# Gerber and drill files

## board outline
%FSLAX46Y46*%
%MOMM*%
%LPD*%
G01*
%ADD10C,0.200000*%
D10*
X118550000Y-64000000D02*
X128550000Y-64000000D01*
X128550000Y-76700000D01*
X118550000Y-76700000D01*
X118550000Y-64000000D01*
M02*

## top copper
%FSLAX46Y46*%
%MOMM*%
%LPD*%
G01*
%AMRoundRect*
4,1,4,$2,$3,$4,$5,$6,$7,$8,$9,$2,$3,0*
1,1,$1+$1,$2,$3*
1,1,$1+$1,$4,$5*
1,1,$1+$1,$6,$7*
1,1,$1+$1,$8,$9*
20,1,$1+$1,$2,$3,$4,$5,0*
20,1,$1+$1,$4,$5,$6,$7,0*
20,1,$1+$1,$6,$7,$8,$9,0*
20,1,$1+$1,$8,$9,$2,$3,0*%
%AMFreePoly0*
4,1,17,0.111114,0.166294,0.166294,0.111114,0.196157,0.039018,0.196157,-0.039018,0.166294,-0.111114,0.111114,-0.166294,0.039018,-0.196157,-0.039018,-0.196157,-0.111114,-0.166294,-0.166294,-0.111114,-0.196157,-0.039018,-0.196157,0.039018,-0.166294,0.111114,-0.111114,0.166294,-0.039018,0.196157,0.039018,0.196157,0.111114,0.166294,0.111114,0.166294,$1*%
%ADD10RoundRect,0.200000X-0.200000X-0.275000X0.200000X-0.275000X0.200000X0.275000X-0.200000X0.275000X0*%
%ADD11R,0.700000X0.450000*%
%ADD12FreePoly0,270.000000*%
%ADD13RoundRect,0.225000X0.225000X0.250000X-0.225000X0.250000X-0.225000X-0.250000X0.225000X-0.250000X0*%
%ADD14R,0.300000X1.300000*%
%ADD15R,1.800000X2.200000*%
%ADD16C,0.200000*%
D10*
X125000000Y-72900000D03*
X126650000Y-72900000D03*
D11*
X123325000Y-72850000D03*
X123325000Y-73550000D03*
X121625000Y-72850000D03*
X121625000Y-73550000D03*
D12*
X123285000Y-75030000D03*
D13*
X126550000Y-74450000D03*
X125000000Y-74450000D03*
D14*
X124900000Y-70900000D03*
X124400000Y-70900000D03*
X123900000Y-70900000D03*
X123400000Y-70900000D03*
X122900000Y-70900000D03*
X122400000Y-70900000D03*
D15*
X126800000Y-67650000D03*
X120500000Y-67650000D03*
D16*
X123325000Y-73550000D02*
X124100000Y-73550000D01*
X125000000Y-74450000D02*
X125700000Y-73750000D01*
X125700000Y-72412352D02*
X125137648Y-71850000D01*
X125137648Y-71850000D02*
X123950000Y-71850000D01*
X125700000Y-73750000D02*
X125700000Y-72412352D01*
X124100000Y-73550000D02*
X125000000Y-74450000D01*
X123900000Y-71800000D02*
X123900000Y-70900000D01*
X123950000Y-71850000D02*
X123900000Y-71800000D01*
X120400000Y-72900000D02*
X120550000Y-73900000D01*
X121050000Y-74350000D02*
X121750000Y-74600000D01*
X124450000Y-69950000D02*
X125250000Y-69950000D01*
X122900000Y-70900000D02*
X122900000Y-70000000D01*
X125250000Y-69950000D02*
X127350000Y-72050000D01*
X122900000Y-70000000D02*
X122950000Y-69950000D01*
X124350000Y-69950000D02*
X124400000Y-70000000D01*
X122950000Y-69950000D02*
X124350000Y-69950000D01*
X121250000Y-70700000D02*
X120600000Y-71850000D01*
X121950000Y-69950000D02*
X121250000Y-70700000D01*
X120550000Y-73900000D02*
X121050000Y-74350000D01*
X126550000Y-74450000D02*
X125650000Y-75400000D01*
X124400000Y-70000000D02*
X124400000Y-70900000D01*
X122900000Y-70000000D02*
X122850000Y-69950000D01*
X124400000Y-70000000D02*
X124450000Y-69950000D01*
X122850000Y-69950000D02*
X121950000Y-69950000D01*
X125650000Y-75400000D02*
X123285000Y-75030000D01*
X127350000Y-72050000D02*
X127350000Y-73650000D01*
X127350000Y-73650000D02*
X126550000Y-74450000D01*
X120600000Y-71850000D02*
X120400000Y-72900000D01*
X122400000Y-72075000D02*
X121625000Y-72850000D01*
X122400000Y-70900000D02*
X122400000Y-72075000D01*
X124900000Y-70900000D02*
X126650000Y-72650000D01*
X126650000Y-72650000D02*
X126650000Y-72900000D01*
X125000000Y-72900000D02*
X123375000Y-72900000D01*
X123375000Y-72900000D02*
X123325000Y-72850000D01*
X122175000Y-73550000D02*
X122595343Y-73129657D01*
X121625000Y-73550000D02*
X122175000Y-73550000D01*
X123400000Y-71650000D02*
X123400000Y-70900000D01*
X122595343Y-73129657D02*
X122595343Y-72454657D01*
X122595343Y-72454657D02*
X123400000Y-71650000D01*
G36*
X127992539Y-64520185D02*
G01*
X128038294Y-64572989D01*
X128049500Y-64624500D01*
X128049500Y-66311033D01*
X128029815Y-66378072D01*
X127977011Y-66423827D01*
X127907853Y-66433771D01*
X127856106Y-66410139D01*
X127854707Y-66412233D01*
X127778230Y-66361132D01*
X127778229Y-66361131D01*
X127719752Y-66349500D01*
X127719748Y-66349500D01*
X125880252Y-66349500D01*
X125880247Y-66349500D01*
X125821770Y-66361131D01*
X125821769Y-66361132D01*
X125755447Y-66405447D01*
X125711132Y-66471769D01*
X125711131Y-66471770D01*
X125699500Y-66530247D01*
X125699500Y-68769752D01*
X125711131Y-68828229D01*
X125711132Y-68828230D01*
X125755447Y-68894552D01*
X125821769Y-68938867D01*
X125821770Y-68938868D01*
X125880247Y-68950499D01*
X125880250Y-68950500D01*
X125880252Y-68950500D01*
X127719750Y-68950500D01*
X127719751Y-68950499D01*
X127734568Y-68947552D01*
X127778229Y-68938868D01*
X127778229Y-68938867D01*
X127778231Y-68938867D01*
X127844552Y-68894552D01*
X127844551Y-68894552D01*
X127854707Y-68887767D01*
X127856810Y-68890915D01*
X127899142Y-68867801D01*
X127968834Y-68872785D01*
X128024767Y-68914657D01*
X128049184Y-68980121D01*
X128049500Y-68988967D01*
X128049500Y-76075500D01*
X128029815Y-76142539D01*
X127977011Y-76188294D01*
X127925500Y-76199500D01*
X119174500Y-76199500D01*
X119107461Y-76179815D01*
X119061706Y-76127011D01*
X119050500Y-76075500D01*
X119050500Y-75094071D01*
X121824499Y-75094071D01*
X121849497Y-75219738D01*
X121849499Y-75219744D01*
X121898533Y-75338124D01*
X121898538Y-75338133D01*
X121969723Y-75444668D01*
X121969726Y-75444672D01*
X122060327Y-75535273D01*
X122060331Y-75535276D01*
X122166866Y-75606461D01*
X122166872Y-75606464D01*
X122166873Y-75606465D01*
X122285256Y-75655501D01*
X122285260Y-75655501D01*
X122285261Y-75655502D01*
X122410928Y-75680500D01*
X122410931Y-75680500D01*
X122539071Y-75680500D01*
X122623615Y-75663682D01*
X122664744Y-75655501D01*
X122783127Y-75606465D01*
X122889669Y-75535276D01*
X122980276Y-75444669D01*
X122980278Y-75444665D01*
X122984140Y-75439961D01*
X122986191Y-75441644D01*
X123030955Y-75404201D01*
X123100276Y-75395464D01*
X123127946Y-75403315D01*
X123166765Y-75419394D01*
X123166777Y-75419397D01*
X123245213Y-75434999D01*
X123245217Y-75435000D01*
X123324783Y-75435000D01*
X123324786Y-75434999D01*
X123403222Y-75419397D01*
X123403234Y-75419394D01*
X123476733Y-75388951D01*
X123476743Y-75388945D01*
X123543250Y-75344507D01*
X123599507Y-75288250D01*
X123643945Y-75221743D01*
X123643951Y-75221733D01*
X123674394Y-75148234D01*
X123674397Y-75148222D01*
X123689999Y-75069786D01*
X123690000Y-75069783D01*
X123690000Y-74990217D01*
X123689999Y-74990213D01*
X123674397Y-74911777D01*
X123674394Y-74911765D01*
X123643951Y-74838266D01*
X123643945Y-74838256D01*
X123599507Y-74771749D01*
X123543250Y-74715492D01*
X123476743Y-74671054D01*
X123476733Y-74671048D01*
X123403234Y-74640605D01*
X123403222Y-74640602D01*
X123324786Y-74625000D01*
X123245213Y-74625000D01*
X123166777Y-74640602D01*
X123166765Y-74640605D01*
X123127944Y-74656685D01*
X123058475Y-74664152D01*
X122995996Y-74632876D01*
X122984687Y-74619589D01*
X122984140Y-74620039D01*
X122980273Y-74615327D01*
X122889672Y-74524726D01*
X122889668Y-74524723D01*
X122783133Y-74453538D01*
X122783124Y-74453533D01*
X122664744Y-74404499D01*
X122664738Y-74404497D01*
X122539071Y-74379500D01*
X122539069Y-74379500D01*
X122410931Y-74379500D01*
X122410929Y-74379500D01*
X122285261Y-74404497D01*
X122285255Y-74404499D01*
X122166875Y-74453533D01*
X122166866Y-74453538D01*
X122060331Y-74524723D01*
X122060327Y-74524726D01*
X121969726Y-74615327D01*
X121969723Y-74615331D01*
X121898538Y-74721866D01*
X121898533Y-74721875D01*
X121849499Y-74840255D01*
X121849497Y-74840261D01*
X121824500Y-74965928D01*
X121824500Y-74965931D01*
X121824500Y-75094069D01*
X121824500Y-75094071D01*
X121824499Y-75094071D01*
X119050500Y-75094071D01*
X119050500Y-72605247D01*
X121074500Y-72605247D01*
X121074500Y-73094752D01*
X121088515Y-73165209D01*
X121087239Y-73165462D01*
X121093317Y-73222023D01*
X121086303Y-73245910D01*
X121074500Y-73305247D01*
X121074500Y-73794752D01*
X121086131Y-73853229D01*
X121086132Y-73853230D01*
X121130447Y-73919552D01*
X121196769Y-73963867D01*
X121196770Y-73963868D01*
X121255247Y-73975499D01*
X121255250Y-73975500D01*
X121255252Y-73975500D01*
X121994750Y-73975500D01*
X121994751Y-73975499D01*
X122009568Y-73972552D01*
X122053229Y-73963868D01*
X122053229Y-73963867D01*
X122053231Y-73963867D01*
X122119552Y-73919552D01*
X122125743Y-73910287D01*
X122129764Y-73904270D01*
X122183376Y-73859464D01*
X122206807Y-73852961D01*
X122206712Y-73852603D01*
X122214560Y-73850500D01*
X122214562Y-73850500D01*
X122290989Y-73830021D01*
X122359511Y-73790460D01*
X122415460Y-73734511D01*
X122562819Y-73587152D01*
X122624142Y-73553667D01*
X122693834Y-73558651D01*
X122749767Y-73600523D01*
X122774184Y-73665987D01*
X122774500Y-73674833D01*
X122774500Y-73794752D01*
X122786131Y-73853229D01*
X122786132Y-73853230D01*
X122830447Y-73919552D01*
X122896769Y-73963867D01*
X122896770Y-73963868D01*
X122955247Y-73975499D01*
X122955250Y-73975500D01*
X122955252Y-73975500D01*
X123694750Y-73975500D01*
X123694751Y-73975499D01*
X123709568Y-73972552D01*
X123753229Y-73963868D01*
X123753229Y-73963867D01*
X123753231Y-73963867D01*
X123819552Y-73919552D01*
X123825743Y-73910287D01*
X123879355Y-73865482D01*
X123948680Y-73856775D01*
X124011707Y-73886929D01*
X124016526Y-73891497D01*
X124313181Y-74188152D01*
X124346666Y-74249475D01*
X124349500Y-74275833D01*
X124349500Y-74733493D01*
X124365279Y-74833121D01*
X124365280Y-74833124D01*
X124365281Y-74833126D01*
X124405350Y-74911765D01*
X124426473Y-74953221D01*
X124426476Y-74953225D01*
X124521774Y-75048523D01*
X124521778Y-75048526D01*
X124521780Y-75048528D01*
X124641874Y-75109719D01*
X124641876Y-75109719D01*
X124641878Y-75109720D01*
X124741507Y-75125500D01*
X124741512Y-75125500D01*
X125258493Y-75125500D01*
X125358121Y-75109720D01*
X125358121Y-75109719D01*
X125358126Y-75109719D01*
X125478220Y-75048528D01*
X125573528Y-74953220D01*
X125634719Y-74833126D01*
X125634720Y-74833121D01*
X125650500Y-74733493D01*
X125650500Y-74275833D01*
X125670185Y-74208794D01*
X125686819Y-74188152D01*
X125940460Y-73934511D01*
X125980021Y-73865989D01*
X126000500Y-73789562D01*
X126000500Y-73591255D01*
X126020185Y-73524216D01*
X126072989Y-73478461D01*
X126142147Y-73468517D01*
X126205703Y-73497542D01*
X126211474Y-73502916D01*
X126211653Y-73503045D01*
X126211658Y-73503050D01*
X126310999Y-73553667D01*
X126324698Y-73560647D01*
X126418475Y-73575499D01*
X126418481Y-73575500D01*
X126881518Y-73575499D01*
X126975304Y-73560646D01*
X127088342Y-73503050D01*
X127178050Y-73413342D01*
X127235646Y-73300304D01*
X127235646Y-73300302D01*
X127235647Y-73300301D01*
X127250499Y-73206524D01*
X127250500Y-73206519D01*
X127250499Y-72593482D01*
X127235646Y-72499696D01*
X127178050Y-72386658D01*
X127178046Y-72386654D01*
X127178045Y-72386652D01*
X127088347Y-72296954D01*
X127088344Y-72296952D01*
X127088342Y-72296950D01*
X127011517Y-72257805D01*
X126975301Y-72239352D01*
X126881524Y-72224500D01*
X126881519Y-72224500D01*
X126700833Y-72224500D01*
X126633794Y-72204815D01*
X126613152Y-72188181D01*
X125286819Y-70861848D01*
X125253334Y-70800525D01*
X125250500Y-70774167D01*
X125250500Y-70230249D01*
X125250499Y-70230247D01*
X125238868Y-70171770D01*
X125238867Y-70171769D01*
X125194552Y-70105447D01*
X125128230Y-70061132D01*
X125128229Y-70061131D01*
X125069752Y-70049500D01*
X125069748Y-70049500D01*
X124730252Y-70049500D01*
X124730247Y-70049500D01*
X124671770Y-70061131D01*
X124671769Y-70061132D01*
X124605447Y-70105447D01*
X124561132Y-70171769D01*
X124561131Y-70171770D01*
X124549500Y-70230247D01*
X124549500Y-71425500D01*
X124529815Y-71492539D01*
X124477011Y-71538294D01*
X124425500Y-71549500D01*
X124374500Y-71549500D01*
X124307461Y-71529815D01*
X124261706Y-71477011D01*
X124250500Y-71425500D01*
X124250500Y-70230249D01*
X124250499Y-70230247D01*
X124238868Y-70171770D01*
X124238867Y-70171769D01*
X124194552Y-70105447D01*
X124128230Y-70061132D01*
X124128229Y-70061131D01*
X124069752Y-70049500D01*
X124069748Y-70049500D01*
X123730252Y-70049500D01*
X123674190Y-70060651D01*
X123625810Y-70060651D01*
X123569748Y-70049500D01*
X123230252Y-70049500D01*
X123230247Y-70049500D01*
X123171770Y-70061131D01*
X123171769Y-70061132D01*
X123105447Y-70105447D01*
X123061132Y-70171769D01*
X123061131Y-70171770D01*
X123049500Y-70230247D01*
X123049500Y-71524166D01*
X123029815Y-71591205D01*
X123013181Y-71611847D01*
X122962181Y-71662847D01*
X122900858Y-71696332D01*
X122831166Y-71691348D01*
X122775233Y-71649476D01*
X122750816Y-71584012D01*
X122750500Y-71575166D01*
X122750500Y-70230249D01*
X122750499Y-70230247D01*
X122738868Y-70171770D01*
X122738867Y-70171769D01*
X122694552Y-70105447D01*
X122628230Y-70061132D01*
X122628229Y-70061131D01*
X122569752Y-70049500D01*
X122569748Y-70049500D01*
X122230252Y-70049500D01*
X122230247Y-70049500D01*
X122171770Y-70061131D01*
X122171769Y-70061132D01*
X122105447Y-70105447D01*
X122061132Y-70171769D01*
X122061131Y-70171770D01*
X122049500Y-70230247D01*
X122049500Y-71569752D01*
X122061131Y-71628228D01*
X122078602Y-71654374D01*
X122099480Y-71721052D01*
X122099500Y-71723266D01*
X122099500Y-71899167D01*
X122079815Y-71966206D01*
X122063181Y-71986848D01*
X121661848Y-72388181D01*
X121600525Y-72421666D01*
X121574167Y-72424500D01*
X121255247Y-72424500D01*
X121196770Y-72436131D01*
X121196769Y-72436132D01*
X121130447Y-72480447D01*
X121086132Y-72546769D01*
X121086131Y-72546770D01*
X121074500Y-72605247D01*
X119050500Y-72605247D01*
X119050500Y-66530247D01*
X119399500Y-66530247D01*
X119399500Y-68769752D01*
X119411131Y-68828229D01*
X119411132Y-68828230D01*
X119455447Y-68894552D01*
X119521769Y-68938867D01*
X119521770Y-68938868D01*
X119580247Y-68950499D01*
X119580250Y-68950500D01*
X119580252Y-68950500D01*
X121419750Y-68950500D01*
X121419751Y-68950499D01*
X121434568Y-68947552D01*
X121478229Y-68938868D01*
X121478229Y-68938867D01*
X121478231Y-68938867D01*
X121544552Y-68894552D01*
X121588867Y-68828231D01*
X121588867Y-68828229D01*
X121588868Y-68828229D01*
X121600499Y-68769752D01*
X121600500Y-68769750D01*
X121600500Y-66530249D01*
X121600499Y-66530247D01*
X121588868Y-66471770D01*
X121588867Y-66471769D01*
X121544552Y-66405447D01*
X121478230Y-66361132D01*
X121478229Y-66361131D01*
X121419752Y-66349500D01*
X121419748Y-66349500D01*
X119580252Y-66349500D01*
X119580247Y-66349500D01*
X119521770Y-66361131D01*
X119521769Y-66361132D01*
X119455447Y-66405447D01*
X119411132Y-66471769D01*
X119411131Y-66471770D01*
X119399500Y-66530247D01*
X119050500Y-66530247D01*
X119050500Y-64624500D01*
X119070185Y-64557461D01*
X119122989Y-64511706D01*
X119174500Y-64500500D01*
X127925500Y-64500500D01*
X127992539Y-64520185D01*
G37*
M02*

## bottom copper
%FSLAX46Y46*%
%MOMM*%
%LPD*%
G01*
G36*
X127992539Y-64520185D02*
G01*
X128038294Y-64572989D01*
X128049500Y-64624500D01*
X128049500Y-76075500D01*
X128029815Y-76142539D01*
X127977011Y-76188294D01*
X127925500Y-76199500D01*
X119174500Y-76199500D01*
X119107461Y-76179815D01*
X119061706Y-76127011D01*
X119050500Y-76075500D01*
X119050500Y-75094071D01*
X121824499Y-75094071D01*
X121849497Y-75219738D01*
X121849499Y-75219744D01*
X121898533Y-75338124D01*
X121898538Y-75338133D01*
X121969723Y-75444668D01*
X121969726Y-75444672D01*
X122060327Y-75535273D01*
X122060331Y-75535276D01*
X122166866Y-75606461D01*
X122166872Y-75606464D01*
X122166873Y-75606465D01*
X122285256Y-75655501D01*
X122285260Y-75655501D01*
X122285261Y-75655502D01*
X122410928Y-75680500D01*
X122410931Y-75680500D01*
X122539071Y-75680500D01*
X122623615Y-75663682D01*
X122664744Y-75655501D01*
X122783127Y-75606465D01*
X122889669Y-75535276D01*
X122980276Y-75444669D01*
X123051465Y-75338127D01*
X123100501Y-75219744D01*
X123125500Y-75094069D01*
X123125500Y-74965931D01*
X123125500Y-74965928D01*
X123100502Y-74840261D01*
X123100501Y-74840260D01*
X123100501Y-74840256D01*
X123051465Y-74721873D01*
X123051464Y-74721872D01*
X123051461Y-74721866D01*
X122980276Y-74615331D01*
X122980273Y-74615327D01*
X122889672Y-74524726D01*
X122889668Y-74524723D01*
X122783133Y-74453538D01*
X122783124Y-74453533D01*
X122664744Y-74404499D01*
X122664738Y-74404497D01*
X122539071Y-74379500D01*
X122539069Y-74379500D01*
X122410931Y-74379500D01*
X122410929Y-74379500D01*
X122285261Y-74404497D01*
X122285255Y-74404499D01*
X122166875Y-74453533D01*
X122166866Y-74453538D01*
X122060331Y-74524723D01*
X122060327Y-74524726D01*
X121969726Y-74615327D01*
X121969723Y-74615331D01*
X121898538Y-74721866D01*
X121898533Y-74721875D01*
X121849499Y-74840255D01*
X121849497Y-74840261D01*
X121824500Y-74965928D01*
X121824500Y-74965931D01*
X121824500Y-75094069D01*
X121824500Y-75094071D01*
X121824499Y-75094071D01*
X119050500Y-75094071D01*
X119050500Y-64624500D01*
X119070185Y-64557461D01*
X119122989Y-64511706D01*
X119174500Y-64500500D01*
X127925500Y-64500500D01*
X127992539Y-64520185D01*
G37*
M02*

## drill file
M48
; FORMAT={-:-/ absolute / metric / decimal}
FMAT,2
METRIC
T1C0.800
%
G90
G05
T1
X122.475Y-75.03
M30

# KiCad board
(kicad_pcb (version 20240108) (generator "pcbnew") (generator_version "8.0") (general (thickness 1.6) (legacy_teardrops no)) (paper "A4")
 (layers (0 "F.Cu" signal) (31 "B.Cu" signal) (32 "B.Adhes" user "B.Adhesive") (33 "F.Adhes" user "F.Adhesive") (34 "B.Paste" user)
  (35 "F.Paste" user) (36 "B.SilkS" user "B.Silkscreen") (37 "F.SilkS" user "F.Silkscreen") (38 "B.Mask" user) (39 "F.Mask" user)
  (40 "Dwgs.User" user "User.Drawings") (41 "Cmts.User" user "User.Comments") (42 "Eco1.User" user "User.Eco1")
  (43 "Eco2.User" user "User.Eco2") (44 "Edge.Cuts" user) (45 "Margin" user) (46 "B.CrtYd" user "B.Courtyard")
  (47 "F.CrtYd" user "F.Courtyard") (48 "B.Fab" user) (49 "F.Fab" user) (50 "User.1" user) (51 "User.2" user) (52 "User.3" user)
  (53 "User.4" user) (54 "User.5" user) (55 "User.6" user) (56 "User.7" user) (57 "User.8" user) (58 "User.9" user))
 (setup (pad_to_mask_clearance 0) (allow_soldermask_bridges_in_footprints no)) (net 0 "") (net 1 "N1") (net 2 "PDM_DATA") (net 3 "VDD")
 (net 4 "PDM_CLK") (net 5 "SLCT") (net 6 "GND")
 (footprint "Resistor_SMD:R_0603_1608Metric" (layer "F.Cu") (at 125.825 72.9)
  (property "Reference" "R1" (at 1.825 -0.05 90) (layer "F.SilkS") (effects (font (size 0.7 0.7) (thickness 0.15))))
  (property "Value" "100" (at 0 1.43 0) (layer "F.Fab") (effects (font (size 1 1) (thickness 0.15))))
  (pad "1" smd roundrect (at -0.825 0) (size 0.8 0.95) (layers "F.Cu" "F.Paste" "F.Mask") (roundrect_rratio 0.25) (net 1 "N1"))
  (pad "2" smd roundrect (at 0.825 0) (size 0.8 0.95) (layers "F.Cu" "F.Paste" "F.Mask") (roundrect_rratio 0.25) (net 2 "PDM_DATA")))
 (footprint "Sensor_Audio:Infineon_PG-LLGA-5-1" (layer "F.Cu") (at 122.475 74.35 -90)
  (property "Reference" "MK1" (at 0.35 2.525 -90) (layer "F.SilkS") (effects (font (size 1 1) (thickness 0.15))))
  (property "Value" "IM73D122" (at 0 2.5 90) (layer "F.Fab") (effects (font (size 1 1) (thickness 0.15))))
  (pad "" smd custom (at -1.5 -0.725 270) (size 0.3 0.3) (layers "F.Paste") (zone_connect 0) (options (clearance outline) (anchor circle))
   (primitives))
  (pad "" smd custom (at -1.5 0.725 270) (size 0.3 0.3) (layers "F.Paste") (zone_connect 0) (options (clearance outline) (anchor circle))
   (primitives))
  (pad "" smd custom (at -0.8 -0.725 270) (size 0.3 0.3) (layers "F.Paste") (zone_connect 0) (options (clearance outline) (anchor circle))
   (primitives))
  (pad "" smd custom (at -0.8 0.725 270) (size 0.3 0.3) (layers "F.Paste") (zone_connect 0) (options (clearance outline) (anchor circle))
   (primitives))
  (pad "" smd custom (at -0.12 0 270) (size 0.3 0.3) (layers "F.Paste") (zone_connect 0) (options (clearance outline) (anchor circle))
   (primitives))
  (pad "" smd custom (at 0.28 -0.693 270) (size 0.3 0.3) (layers "F.Paste") (zone_connect 0) (options (clearance outline) (anchor circle))
   (primitives))
  (pad "" smd custom (at 0.28 0.693 270) (size 0.3 0.3) (layers "F.Paste") (zone_connect 0) (options (clearance outline) (anchor circle))
   (primitives))
  (pad "" np_thru_hole circle (at 0.68 0 270) (size 0.8 0.8) (drill 0.8) (layers "*.Cu" "*.Mask"))
  (pad "" smd custom (at 1.08 -0.693 270) (size 0.3 0.3) (layers "F.Paste") (zone_connect 0) (options (clearance outline) (anchor circle))
   (primitives))
  (pad "" smd custom (at 1.08 0.693 270) (size 0.3 0.3) (layers "F.Paste") (zone_connect 0) (options (clearance outline) (anchor circle))
   (primitives))
  (pad "" smd custom (at 1.48 0 270) (size 0.3 0.3) (layers "F.Paste") (zone_connect 0) (options (clearance outline) (anchor circle))
   (primitives))
  (pad "1" smd rect (at -1.5 -0.85 270) (size 0.45 0.7) (layers "F.Cu" "F.Mask") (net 1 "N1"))
  (pad "2" smd rect (at -0.8 -0.85 270) (size 0.45 0.7) (layers "F.Cu" "F.Mask") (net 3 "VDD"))
  (pad "3" smd rect (at -1.5 0.85 270) (size 0.45 0.7) (layers "F.Cu" "F.Mask") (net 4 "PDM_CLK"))
  (pad "4" smd rect (at -0.8 0.85 270) (size 0.45 0.7) (layers "F.Cu" "F.Mask") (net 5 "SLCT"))
  (pad "5" smd custom (at 0.68 -0.81 270) (size 0.4 0.4) (layers "F.Cu" "F.Mask") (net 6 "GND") (zone_connect 0)
   (options (clearance outline) (anchor circle)) (primitives)))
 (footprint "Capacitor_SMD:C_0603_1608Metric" (layer "F.Cu") (at 125.775 74.45 180)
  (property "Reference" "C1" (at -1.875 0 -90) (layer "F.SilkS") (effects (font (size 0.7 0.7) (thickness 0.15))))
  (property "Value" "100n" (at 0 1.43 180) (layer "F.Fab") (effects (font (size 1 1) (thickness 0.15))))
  (pad "1" smd roundrect (at -0.775 0 180) (size 0.9 0.95) (layers "F.Cu" "F.Paste" "F.Mask") (roundrect_rratio 0.25) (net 6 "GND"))
  (pad "2" smd roundrect (at 0.775 0 180) (size 0.9 0.95) (layers "F.Cu" "F.Paste" "F.Mask") (roundrect_rratio 0.25) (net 3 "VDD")))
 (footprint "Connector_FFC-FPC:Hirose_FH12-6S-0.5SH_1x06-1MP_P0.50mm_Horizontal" (layer "F.Cu") (at 123.65 69.05 180)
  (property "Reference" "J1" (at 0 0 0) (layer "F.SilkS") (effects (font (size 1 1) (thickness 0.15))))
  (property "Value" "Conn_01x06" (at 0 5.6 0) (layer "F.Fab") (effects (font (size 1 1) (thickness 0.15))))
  (pad "1" smd rect (at -1.25 -1.85 180) (size 0.3 1.3) (layers "F.Cu" "F.Paste" "F.Mask") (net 2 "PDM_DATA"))
  (pad "2" smd rect (at -0.75 -1.85 180) (size 0.3 1.3) (layers "F.Cu" "F.Paste" "F.Mask") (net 6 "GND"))
  (pad "3" smd rect (at -0.25 -1.85 180) (size 0.3 1.3) (layers "F.Cu" "F.Paste" "F.Mask") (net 3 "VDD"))
  (pad "4" smd rect (at 0.25 -1.85 180) (size 0.3 1.3) (layers "F.Cu" "F.Paste" "F.Mask") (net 5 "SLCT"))
  (pad "5" smd rect (at 0.75 -1.85 180) (size 0.3 1.3) (layers "F.Cu" "F.Paste" "F.Mask") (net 6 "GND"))
  (pad "6" smd rect (at 1.25 -1.85 180) (size 0.3 1.3) (layers "F.Cu" "F.Paste" "F.Mask") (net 4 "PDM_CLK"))
  (pad "MP" smd rect (at -3.15 1.4 180) (size 1.8 2.2) (layers "F.Cu" "F.Paste" "F.Mask"))
  (pad "MP" smd rect (at 3.15 1.4 180) (size 1.8 2.2) (layers "F.Cu" "F.Paste" "F.Mask")))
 (gr_rect (start 118.55 64) (end 128.55 76.7) (stroke (width 0.2) (type default)) (fill none) (layer "Edge.Cuts"))
 (segment (start 123.325 73.55) (end 124.1 73.55) (width 0.2) (layer "F.Cu") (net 3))
 (segment (start 125 74.45) (end 125.7 73.75) (width 0.2) (layer "F.Cu") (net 3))
 (segment (start 125.7 72.412352) (end 125.137648 71.85) (width 0.2) (layer "F.Cu") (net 3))
 (segment (start 125.137648 71.85) (end 123.95 71.85) (width 0.2) (layer "F.Cu") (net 3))
 (segment (start 125.7 73.75) (end 125.7 72.412352) (width 0.2) (layer "F.Cu") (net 3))
 (segment (start 124.1 73.55) (end 125 74.45) (width 0.2) (layer "F.Cu") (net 3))
 (segment (start 123.9 71.8) (end 123.9 70.9) (width 0.2) (layer "F.Cu") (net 3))
 (segment (start 123.95 71.85) (end 123.9 71.8) (width 0.2) (layer "F.Cu") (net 3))
 (segment (start 120.4 72.9) (end 120.55 73.9) (width 0.2) (layer "F.Cu") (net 6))
 (segment (start 121.05 74.35) (end 121.75 74.6) (width 0.2) (layer "F.Cu") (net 6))
 (segment (start 124.45 69.95) (end 125.25 69.95) (width 0.2) (layer "F.Cu") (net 6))
 (segment (start 122.9 70.9) (end 122.9 70) (width 0.2) (layer "F.Cu") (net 6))
 (segment (start 125.25 69.95) (end 127.35 72.05) (width 0.2) (layer "F.Cu") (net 6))
 (segment (start 122.9 70) (end 122.95 69.95) (width 0.2) (layer "F.Cu") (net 6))
 (segment (start 124.35 69.95) (end 124.4 70) (width 0.2) (layer "F.Cu") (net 6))
 (segment (start 122.95 69.95) (end 124.35 69.95) (width 0.2) (layer "F.Cu") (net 6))
 (segment (start 121.25 70.7) (end 120.6 71.85) (width 0.2) (layer "F.Cu") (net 6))
 (segment (start 121.95 69.95) (end 121.25 70.7) (width 0.2) (layer "F.Cu") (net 6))
 (segment (start 120.55 73.9) (end 121.05 74.35) (width 0.2) (layer "F.Cu") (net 6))
 (segment (start 126.55 74.45) (end 125.65 75.4) (width 0.2) (layer "F.Cu") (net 6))
 (segment (start 124.4 70) (end 124.4 70.9) (width 0.2) (layer "F.Cu") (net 6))
 (segment (start 122.9 70) (end 122.85 69.95) (width 0.2) (layer "F.Cu") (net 6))
 (segment (start 124.4 70) (end 124.45 69.95) (width 0.2) (layer "F.Cu") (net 6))
 (segment (start 122.85 69.95) (end 121.95 69.95) (width 0.2) (layer "F.Cu") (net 6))
 (segment (start 125.65 75.4) (end 123.285 75.03) (width 0.2) (layer "F.Cu") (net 6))
 (segment (start 127.35 72.05) (end 127.35 73.65) (width 0.2) (layer "F.Cu") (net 6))
 (segment (start 127.35 73.65) (end 126.55 74.45) (width 0.2) (layer "F.Cu") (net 6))
 (segment (start 120.6 71.85) (end 120.4 72.9) (width 0.2) (layer "F.Cu") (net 6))
 (segment (start 122.4 72.075) (end 121.625 72.85) (width 0.2) (layer "F.Cu") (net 4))
 (segment (start 122.4 70.9) (end 122.4 72.075) (width 0.2) (layer "F.Cu") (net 4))
 (segment (start 124.9 70.9) (end 126.65 72.65) (width 0.2) (layer "F.Cu") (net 2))
 (segment (start 126.65 72.65) (end 126.65 72.9) (width 0.2) (layer "F.Cu") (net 2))
 (segment (start 125 72.9) (end 123.375 72.9) (width 0.2) (layer "F.Cu") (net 1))
 (segment (start 123.375 72.9) (end 123.325 72.85) (width 0.2) (layer "F.Cu") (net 1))
 (segment (start 122.175 73.55) (end 122.595343 73.129657) (width 0.2) (layer "F.Cu") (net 5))
 (segment (start 121.625 73.55) (end 122.175 73.55) (width 0.2) (layer "F.Cu") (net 5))
 (segment (start 123.4 71.65) (end 123.4 70.9) (width 0.2) (layer "F.Cu") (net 5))
 (segment (start 122.595343 73.129657) (end 122.595343 72.454657) (width 0.2) (layer "F.Cu") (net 5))
 (segment (start 122.595343 72.454657) (end 123.4 71.65) (width 0.2) (layer "F.Cu") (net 5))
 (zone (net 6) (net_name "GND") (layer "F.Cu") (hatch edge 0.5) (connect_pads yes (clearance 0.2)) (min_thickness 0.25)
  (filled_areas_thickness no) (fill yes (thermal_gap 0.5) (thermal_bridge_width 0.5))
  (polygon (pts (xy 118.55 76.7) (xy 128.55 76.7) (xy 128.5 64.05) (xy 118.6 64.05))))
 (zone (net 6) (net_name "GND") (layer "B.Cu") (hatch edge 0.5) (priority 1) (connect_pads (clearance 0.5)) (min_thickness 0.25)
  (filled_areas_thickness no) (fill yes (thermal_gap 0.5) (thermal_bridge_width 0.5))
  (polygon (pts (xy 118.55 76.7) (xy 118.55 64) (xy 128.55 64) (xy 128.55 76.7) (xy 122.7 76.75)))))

